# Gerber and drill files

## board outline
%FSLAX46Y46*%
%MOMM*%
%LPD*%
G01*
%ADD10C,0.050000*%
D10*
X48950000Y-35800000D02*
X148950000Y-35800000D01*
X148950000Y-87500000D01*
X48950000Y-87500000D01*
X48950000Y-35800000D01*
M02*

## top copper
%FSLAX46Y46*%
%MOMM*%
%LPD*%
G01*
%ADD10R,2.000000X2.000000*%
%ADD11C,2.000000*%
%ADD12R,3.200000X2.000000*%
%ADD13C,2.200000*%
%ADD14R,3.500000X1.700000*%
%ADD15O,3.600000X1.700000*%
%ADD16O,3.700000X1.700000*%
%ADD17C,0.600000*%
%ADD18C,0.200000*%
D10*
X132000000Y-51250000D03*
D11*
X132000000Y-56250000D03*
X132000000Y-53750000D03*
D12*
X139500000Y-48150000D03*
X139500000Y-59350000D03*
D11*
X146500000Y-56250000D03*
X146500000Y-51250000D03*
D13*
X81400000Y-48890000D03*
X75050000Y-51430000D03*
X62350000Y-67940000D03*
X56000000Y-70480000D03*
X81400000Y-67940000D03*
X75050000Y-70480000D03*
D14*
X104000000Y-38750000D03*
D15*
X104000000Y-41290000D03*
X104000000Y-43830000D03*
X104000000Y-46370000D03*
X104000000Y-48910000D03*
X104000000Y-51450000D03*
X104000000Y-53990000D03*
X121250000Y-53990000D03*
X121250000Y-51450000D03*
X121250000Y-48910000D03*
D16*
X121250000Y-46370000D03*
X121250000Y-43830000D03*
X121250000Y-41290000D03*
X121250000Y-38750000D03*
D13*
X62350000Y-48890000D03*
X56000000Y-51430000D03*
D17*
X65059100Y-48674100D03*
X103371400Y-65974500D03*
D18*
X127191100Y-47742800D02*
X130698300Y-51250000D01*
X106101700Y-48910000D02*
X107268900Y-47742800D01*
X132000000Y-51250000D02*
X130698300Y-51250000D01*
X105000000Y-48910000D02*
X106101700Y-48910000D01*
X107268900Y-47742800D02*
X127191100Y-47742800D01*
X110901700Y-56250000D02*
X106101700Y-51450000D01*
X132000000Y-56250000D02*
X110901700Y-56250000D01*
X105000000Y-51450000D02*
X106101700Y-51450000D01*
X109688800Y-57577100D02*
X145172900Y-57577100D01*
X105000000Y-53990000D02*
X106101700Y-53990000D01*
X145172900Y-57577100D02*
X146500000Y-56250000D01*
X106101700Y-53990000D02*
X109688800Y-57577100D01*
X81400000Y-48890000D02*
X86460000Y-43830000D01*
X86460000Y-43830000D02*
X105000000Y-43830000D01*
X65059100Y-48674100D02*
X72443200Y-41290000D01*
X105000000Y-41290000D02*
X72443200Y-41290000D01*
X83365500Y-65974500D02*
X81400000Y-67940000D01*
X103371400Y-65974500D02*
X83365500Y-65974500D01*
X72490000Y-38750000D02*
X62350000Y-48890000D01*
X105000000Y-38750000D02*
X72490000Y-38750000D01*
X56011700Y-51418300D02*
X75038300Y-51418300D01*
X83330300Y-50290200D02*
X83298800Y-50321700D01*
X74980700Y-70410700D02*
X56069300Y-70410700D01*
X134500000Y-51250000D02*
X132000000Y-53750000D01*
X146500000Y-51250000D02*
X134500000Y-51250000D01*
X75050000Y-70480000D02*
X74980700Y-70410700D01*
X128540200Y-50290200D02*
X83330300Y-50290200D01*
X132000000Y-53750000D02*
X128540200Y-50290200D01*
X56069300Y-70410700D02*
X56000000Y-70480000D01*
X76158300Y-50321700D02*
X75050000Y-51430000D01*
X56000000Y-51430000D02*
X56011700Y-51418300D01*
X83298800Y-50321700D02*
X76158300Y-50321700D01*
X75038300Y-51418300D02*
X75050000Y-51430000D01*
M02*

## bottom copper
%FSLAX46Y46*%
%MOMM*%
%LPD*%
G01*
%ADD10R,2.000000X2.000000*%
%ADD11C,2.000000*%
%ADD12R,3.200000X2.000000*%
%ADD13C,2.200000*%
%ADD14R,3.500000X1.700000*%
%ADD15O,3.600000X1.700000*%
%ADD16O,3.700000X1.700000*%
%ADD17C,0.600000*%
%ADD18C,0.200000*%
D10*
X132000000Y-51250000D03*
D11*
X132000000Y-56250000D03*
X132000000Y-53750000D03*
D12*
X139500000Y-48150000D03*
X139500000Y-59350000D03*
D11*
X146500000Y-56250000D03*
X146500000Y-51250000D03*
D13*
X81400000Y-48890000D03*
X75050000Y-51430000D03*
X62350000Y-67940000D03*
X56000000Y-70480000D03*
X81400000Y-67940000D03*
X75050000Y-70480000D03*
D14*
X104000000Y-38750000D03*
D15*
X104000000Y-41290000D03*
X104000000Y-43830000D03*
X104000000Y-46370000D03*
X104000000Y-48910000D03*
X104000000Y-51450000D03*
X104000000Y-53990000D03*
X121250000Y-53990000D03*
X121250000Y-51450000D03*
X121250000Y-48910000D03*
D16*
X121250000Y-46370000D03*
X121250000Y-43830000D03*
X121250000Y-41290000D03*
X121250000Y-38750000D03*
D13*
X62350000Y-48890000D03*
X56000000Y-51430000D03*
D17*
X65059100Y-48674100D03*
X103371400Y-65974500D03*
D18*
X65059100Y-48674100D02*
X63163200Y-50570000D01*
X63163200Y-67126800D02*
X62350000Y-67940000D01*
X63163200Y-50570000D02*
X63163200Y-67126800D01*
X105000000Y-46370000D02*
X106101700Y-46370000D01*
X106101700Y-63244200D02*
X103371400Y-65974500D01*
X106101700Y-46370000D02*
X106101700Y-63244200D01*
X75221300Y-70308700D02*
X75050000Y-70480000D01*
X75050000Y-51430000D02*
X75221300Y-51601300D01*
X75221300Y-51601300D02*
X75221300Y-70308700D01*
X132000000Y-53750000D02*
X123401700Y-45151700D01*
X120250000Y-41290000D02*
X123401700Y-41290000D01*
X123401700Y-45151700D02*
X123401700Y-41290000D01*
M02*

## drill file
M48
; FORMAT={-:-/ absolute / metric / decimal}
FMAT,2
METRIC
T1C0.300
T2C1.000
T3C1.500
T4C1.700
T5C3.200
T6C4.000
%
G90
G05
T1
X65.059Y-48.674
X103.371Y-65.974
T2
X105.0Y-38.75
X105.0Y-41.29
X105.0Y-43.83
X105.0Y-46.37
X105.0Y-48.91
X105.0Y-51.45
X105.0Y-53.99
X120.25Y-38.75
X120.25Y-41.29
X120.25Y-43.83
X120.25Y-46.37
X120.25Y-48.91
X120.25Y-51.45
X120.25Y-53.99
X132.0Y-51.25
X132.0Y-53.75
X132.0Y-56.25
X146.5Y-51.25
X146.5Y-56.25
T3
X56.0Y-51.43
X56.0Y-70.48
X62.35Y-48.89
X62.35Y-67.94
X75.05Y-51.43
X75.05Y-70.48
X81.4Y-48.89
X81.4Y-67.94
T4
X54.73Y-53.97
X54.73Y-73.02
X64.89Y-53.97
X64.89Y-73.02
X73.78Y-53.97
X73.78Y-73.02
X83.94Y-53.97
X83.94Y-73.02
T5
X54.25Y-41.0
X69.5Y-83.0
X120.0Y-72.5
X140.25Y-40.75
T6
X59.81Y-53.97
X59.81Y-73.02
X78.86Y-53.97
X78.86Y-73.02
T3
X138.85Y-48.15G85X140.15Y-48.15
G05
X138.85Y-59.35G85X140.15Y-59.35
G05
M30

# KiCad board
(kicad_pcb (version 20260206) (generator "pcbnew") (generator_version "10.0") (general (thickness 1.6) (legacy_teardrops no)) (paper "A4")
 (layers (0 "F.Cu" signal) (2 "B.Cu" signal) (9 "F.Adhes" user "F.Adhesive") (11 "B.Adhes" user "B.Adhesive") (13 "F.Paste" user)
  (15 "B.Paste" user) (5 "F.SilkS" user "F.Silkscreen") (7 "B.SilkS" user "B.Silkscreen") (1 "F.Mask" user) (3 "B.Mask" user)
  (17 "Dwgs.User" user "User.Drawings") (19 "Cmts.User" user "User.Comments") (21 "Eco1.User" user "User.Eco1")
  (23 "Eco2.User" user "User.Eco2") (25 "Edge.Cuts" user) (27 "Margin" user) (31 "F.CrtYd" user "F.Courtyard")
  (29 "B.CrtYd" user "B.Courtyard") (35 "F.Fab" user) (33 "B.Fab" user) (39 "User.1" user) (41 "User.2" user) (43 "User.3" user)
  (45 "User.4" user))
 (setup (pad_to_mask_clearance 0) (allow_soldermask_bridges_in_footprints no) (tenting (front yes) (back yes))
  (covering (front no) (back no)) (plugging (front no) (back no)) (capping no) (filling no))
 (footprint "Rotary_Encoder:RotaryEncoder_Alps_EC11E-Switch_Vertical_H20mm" (layer "F.Cu") (at 132 51.25)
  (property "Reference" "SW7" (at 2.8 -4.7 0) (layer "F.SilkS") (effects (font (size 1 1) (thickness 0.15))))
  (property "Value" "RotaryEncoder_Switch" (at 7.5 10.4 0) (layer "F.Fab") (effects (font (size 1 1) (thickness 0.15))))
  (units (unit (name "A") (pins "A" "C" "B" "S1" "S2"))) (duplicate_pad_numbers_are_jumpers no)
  (pad "A" thru_hole rect (at 0 0) (size 2 2) (drill 1) (layers "*.Cu" "*.Mask") (remove_unused_layers no) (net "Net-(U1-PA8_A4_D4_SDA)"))
  (pad "B" thru_hole circle (at 0 5) (size 2 2) (drill 1) (layers "*.Cu" "*.Mask") (remove_unused_layers no) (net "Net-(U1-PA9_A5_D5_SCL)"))
  (pad "C" thru_hole circle (at 0 2.5) (size 2 2) (drill 1) (layers "*.Cu" "*.Mask") (remove_unused_layers no) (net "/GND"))
  (pad "MP" thru_hole rect (at 7.5 -3.1) (size 3.2 2) (drill oval 2.8 1.5) (layers "*.Cu" "*.Mask") (remove_unused_layers no))
  (pad "MP" thru_hole rect (at 7.5 8.1) (size 3.2 2) (drill oval 2.8 1.5) (layers "*.Cu" "*.Mask") (remove_unused_layers no))
  (pad "S1" thru_hole circle (at 14.5 5) (size 2 2) (drill 1) (layers "*.Cu" "*.Mask") (remove_unused_layers no)
   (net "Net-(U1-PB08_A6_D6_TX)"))
  (pad "S2" thru_hole circle (at 14.5 0) (size 2 2) (drill 1) (layers "*.Cu" "*.Mask") (remove_unused_layers no) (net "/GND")))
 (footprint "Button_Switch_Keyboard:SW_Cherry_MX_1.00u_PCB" (layer "F.Cu") (at 81.4 48.89)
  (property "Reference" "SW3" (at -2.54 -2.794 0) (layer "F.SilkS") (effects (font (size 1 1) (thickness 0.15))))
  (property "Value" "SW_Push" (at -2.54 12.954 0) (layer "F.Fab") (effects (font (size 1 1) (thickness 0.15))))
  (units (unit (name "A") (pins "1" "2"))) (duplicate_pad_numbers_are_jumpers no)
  (pad "" np_thru_hole circle (at -7.62 5.08) (size 1.7 1.7) (drill 1.7) (layers "*.Cu" "*.Mask"))
  (pad "" np_thru_hole circle (at -2.54 5.08) (size 4 4) (drill 4) (layers "*.Cu" "*.Mask"))
  (pad "" np_thru_hole circle (at 2.54 5.08) (size 1.7 1.7) (drill 1.7) (layers "*.Cu" "*.Mask"))
  (pad "1" thru_hole circle (at 0 0) (size 2.2 2.2) (drill 1.5) (layers "*.Cu" "*.Mask") (remove_unused_layers no)
   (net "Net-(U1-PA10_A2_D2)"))
  (pad "2" thru_hole circle (at -6.35 2.54) (size 2.2 2.2) (drill 1.5) (layers "*.Cu" "*.Mask") (remove_unused_layers no) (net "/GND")))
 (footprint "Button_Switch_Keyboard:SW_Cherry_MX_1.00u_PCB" (layer "F.Cu") (at 62.35 67.94)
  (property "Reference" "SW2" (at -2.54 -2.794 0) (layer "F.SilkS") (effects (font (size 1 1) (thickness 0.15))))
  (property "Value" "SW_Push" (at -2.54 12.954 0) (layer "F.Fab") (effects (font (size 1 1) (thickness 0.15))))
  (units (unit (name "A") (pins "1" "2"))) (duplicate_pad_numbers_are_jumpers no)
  (pad "" np_thru_hole circle (at -7.62 5.08) (size 1.7 1.7) (drill 1.7) (layers "*.Cu" "*.Mask"))
  (pad "" np_thru_hole circle (at -2.54 5.08) (size 4 4) (drill 4) (layers "*.Cu" "*.Mask"))
  (pad "" np_thru_hole circle (at 2.54 5.08) (size 1.7 1.7) (drill 1.7) (layers "*.Cu" "*.Mask"))
  (pad "1" thru_hole circle (at 0 0) (size 2.2 2.2) (drill 1.5) (layers "*.Cu" "*.Mask") (remove_unused_layers no)
   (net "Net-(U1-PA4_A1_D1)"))
  (pad "2" thru_hole circle (at -6.35 2.54) (size 2.2 2.2) (drill 1.5) (layers "*.Cu" "*.Mask") (remove_unused_layers no) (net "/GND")))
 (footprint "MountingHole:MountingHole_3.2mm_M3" (layer "F.Cu") (at 140.25 40.75)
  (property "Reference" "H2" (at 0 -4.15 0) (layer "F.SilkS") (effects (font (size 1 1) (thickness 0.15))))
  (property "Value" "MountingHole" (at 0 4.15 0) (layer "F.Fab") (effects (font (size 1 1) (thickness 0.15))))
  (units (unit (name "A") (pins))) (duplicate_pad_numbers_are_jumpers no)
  (pad "" np_thru_hole circle (at 0 0) (size 3.2 3.2) (drill 3.2) (layers "*.Cu" "*.Mask")))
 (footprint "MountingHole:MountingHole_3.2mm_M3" (layer "F.Cu") (at 54.25 41)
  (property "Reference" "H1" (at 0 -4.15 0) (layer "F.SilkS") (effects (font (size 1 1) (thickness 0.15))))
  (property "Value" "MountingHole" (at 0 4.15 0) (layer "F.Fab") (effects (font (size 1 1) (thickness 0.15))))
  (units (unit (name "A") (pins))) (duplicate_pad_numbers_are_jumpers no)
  (pad "" np_thru_hole circle (at 0 0) (size 3.2 3.2) (drill 3.2) (layers "*.Cu" "*.Mask")))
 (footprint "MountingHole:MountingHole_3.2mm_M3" (layer "F.Cu") (at 120 72.5)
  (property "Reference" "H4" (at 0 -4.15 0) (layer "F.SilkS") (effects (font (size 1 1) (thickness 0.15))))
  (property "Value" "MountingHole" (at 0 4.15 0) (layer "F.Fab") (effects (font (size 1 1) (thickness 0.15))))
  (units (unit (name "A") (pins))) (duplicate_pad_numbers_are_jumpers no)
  (pad "" np_thru_hole circle (at 0 0) (size 3.2 3.2) (drill 3.2) (layers "*.Cu" "*.Mask")))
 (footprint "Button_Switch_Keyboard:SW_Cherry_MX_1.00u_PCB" (layer "F.Cu") (at 81.4 67.94)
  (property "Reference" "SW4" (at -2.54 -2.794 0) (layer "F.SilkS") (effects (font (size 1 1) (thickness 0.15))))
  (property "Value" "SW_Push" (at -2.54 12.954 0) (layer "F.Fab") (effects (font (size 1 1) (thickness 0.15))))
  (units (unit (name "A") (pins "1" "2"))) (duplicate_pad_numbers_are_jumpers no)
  (pad "" np_thru_hole circle (at -7.62 5.08) (size 1.7 1.7) (drill 1.7) (layers "*.Cu" "*.Mask"))
  (pad "" np_thru_hole circle (at -2.54 5.08) (size 4 4) (drill 4) (layers "*.Cu" "*.Mask"))
  (pad "" np_thru_hole circle (at 2.54 5.08) (size 1.7 1.7) (drill 1.7) (layers "*.Cu" "*.Mask"))
  (pad "1" thru_hole circle (at 0 0) (size 2.2 2.2) (drill 1.5) (layers "*.Cu" "*.Mask") (remove_unused_layers no)
   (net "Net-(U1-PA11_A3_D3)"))
  (pad "2" thru_hole circle (at -6.35 2.54) (size 2.2 2.2) (drill 1.5) (layers "*.Cu" "*.Mask") (remove_unused_layers no) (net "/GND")))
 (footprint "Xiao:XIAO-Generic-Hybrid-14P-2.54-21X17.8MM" (layer "F.Cu") (at 112.625 46.37)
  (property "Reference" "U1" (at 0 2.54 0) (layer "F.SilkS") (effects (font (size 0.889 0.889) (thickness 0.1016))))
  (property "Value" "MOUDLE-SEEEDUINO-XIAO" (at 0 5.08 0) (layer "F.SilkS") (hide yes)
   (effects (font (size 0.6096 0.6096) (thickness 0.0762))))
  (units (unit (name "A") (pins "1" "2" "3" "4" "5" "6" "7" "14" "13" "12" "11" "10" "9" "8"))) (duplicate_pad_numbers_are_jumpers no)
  (pad "1" thru_hole rect (at -7.625 -7.62) (size 3.5 1.7) (drill 1 (offset -1 0)) (layers "*.Cu" "*.Mask") (remove_unused_layers no)
   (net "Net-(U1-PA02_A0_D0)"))
  (pad "2" thru_hole oval (at -7.625 -5.08) (size 3.6 1.7) (drill 1 (offset -1 0)) (layers "*.Cu" "*.Mask") (remove_unused_layers no)
   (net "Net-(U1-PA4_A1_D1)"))
  (pad "3" thru_hole oval (at -7.625 -2.54) (size 3.6 1.7) (drill 1 (offset -1 0)) (layers "*.Cu" "*.Mask") (remove_unused_layers no)
   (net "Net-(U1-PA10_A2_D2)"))
  (pad "4" thru_hole oval (at -7.625 0) (size 3.6 1.7) (drill 1 (offset -1 0)) (layers "*.Cu" "*.Mask") (remove_unused_layers no)
   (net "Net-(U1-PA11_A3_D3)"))
  (pad "5" thru_hole oval (at -7.625 2.54) (size 3.6 1.7) (drill 1 (offset -1 0)) (layers "*.Cu" "*.Mask") (remove_unused_layers no)
   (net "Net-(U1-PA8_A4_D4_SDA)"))
  (pad "6" thru_hole oval (at -7.625 5.08 180) (size 3.6 1.7) (drill 1 (offset 1 0)) (layers "*.Cu" "*.Mask") (remove_unused_layers no)
   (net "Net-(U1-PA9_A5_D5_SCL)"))
  (pad "7" thru_hole oval (at -7.625 7.62) (size 3.6 1.7) (drill 1 (offset -1 0)) (layers "*.Cu" "*.Mask") (remove_unused_layers no)
   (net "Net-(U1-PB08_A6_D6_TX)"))
  (pad "8" thru_hole oval (at 7.625 7.62) (size 3.6 1.7) (drill 1 (offset 1 0)) (layers "*.Cu" "*.Mask") (remove_unused_layers no)
   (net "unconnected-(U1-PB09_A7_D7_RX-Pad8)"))
  (pad "9" thru_hole oval (at 7.625 5.08) (size 3.6 1.7) (drill 1 (offset 1 0)) (layers "*.Cu" "*.Mask") (remove_unused_layers no)
   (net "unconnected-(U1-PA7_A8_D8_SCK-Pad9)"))
  (pad "10" thru_hole oval (at 7.625 2.54) (size 3.6 1.7) (drill 1 (offset 1 0)) (layers "*.Cu" "*.Mask") (remove_unused_layers no)
   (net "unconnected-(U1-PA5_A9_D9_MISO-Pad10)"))
  (pad "11" thru_hole oval (at 7.625 0) (size 3.7 1.7) (drill 1 (offset 1 0)) (layers "*.Cu" "*.Mask") (remove_unused_layers no)
   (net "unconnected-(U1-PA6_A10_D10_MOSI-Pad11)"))
  (pad "12" thru_hole oval (at 7.625 -2.54) (size 3.7 1.7) (drill 1 (offset 1 0)) (layers "*.Cu" "*.Mask") (remove_unused_layers no)
   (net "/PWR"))
  (pad "13" thru_hole oval (at 7.625 -5.08) (size 3.7 1.7) (drill 1 (offset 1 0)) (layers "*.Cu" "*.Mask") (remove_unused_layers no)
   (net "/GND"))
  (pad "14" thru_hole oval (at 7.625 -7.62) (size 3.7 1.7) (drill 1 (offset 1 0)) (layers "*.Cu" "*.Mask") (remove_unused_layers no)
   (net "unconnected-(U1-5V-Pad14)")))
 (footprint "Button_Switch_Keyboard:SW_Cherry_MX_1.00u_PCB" (layer "F.Cu") (at 62.35 48.89)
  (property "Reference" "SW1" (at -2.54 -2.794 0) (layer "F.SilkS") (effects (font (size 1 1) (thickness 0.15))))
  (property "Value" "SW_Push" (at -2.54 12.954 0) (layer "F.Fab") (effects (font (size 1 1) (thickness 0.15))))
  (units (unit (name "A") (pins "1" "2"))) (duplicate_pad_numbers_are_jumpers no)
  (pad "" np_thru_hole circle (at -7.62 5.08) (size 1.7 1.7) (drill 1.7) (layers "*.Cu" "*.Mask"))
  (pad "" np_thru_hole circle (at -2.54 5.08) (size 4 4) (drill 4) (layers "*.Cu" "*.Mask"))
  (pad "" np_thru_hole circle (at 2.54 5.08) (size 1.7 1.7) (drill 1.7) (layers "*.Cu" "*.Mask"))
  (pad "1" thru_hole circle (at 0 0) (size 2.2 2.2) (drill 1.5) (layers "*.Cu" "*.Mask") (remove_unused_layers no)
   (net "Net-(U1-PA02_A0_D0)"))
  (pad "2" thru_hole circle (at -6.35 2.54) (size 2.2 2.2) (drill 1.5) (layers "*.Cu" "*.Mask") (remove_unused_layers no) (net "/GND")))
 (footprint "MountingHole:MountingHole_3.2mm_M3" (layer "F.Cu") (at 69.5 83)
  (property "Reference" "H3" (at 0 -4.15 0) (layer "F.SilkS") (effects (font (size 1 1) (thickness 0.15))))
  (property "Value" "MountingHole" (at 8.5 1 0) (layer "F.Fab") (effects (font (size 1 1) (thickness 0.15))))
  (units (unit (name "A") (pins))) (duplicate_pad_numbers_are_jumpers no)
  (pad "" np_thru_hole circle (at 0 0) (size 3.2 3.2) (drill 3.2) (layers "*.Cu" "*.Mask")))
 (gr_rect (start 48.95 35.8) (end 148.95 87.5) (stroke (width 0.05) (type solid)) (fill no) (layer "Edge.Cuts"))
 (segment (start 127.1911 47.7428) (end 130.6983 51.25) (width 0.2) (layer "F.Cu") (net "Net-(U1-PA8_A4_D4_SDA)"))
 (segment (start 106.1017 48.91) (end 107.2689 47.7428) (width 0.2) (layer "F.Cu") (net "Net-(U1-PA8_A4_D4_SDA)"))
 (segment (start 132 51.25) (end 130.6983 51.25) (width 0.2) (layer "F.Cu") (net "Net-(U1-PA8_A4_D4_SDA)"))
 (segment (start 105 48.91) (end 106.1017 48.91) (width 0.2) (layer "F.Cu") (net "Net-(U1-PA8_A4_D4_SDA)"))
 (segment (start 107.2689 47.7428) (end 127.1911 47.7428) (width 0.2) (layer "F.Cu") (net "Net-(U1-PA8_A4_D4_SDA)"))
 (segment (start 110.9017 56.25) (end 106.1017 51.45) (width 0.2) (layer "F.Cu") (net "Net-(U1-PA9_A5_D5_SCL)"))
 (segment (start 132 56.25) (end 110.9017 56.25) (width 0.2) (layer "F.Cu") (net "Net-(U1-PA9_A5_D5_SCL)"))
 (segment (start 105 51.45) (end 106.1017 51.45) (width 0.2) (layer "F.Cu") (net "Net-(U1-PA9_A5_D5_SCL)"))
 (segment (start 109.6888 57.5771) (end 145.1729 57.5771) (width 0.2) (layer "F.Cu") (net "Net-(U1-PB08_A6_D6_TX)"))
 (segment (start 105 53.99) (end 106.1017 53.99) (width 0.2) (layer "F.Cu") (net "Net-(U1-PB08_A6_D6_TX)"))
 (segment (start 145.1729 57.5771) (end 146.5 56.25) (width 0.2) (layer "F.Cu") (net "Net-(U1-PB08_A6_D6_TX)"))
 (segment (start 106.1017 53.99) (end 109.6888 57.5771) (width 0.2) (layer "F.Cu") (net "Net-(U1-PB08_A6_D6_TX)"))
 (segment (start 81.4 48.89) (end 86.46 43.83) (width 0.2) (layer "F.Cu") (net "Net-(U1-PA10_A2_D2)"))
 (segment (start 86.46 43.83) (end 105 43.83) (width 0.2) (layer "F.Cu") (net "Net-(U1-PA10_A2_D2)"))
 (segment (start 65.0591 48.6741) (end 72.4432 41.29) (width 0.2) (layer "F.Cu") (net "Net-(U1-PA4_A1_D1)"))
 (segment (start 105 41.29) (end 72.4432 41.29) (width 0.2) (layer "F.Cu") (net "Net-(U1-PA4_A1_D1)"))
 (via (at 65.0591 48.6741) (size 0.6) (drill 0.3) (layers "F.Cu" "B.Cu") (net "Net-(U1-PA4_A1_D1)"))
 (segment (start 65.0591 48.6741) (end 63.1632 50.57) (width 0.2) (layer "B.Cu") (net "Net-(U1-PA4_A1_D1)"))
 (segment (start 63.1632 67.1268) (end 62.35 67.94) (width 0.2) (layer "B.Cu") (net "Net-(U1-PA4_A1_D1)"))
 (segment (start 63.1632 50.57) (end 63.1632 67.1268) (width 0.2) (layer "B.Cu") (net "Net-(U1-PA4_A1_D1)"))
 (segment (start 83.3655 65.9745) (end 81.4 67.94) (width 0.2) (layer "F.Cu") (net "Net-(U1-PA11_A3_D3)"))
 (segment (start 103.3714 65.9745) (end 83.3655 65.9745) (width 0.2) (layer "F.Cu") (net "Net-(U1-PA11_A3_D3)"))
 (via (at 103.3714 65.9745) (size 0.6) (drill 0.3) (layers "F.Cu" "B.Cu") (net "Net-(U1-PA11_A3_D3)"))
 (segment (start 105 46.37) (end 106.1017 46.37) (width 0.2) (layer "B.Cu") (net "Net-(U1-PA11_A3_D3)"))
 (segment (start 106.1017 63.2442) (end 103.3714 65.9745) (width 0.2) (layer "B.Cu") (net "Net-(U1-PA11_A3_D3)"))
 (segment (start 106.1017 46.37) (end 106.1017 63.2442) (width 0.2) (layer "B.Cu") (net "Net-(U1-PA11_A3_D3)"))
 (segment (start 72.49 38.75) (end 62.35 48.89) (width 0.2) (layer "F.Cu") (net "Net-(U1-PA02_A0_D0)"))
 (segment (start 105 38.75) (end 72.49 38.75) (width 0.2) (layer "F.Cu") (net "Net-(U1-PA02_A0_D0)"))
 (segment (start 56.0117 51.4183) (end 75.0383 51.4183) (width 0.2) (layer "F.Cu") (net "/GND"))
 (segment (start 83.3303 50.2902) (end 83.2988 50.3217) (width 0.2) (layer "F.Cu") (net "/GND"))
 (segment (start 74.9807 70.4107) (end 56.0693 70.4107) (width 0.2) (layer "F.Cu") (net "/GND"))
 (segment (start 134.5 51.25) (end 132 53.75) (width 0.2) (layer "F.Cu") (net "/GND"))
 (segment (start 146.5 51.25) (end 134.5 51.25) (width 0.2) (layer "F.Cu") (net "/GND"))
 (segment (start 75.05 70.48) (end 74.9807 70.4107) (width 0.2) (layer "F.Cu") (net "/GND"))
 (segment (start 128.5402 50.2902) (end 83.3303 50.2902) (width 0.2) (layer "F.Cu") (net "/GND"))
 (segment (start 132 53.75) (end 128.5402 50.2902) (width 0.2) (layer "F.Cu") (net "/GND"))
 (segment (start 56.0693 70.4107) (end 56 70.48) (width 0.2) (layer "F.Cu") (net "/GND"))
 (segment (start 76.1583 50.3217) (end 75.05 51.43) (width 0.2) (layer "F.Cu") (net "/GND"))
 (segment (start 56 51.43) (end 56.0117 51.4183) (width 0.2) (layer "F.Cu") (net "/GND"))
 (segment (start 83.2988 50.3217) (end 76.1583 50.3217) (width 0.2) (layer "F.Cu") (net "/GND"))
 (segment (start 75.0383 51.4183) (end 75.05 51.43) (width 0.2) (layer "F.Cu") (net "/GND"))
 (segment (start 75.2213 70.3087) (end 75.05 70.48) (width 0.2) (layer "B.Cu") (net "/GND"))
 (segment (start 75.05 51.43) (end 75.2213 51.6013) (width 0.2) (layer "B.Cu") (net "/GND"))
 (segment (start 75.2213 51.6013) (end 75.2213 70.3087) (width 0.2) (layer "B.Cu") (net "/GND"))
 (segment (start 132 53.75) (end 123.4017 45.1517) (width 0.2) (layer "B.Cu") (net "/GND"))
 (segment (start 120.25 41.29) (end 123.4017 41.29) (width 0.2) (layer "B.Cu") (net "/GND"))
 (segment (start 123.4017 45.1517) (end 123.4017 41.29) (width 0.2) (layer "B.Cu") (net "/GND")))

